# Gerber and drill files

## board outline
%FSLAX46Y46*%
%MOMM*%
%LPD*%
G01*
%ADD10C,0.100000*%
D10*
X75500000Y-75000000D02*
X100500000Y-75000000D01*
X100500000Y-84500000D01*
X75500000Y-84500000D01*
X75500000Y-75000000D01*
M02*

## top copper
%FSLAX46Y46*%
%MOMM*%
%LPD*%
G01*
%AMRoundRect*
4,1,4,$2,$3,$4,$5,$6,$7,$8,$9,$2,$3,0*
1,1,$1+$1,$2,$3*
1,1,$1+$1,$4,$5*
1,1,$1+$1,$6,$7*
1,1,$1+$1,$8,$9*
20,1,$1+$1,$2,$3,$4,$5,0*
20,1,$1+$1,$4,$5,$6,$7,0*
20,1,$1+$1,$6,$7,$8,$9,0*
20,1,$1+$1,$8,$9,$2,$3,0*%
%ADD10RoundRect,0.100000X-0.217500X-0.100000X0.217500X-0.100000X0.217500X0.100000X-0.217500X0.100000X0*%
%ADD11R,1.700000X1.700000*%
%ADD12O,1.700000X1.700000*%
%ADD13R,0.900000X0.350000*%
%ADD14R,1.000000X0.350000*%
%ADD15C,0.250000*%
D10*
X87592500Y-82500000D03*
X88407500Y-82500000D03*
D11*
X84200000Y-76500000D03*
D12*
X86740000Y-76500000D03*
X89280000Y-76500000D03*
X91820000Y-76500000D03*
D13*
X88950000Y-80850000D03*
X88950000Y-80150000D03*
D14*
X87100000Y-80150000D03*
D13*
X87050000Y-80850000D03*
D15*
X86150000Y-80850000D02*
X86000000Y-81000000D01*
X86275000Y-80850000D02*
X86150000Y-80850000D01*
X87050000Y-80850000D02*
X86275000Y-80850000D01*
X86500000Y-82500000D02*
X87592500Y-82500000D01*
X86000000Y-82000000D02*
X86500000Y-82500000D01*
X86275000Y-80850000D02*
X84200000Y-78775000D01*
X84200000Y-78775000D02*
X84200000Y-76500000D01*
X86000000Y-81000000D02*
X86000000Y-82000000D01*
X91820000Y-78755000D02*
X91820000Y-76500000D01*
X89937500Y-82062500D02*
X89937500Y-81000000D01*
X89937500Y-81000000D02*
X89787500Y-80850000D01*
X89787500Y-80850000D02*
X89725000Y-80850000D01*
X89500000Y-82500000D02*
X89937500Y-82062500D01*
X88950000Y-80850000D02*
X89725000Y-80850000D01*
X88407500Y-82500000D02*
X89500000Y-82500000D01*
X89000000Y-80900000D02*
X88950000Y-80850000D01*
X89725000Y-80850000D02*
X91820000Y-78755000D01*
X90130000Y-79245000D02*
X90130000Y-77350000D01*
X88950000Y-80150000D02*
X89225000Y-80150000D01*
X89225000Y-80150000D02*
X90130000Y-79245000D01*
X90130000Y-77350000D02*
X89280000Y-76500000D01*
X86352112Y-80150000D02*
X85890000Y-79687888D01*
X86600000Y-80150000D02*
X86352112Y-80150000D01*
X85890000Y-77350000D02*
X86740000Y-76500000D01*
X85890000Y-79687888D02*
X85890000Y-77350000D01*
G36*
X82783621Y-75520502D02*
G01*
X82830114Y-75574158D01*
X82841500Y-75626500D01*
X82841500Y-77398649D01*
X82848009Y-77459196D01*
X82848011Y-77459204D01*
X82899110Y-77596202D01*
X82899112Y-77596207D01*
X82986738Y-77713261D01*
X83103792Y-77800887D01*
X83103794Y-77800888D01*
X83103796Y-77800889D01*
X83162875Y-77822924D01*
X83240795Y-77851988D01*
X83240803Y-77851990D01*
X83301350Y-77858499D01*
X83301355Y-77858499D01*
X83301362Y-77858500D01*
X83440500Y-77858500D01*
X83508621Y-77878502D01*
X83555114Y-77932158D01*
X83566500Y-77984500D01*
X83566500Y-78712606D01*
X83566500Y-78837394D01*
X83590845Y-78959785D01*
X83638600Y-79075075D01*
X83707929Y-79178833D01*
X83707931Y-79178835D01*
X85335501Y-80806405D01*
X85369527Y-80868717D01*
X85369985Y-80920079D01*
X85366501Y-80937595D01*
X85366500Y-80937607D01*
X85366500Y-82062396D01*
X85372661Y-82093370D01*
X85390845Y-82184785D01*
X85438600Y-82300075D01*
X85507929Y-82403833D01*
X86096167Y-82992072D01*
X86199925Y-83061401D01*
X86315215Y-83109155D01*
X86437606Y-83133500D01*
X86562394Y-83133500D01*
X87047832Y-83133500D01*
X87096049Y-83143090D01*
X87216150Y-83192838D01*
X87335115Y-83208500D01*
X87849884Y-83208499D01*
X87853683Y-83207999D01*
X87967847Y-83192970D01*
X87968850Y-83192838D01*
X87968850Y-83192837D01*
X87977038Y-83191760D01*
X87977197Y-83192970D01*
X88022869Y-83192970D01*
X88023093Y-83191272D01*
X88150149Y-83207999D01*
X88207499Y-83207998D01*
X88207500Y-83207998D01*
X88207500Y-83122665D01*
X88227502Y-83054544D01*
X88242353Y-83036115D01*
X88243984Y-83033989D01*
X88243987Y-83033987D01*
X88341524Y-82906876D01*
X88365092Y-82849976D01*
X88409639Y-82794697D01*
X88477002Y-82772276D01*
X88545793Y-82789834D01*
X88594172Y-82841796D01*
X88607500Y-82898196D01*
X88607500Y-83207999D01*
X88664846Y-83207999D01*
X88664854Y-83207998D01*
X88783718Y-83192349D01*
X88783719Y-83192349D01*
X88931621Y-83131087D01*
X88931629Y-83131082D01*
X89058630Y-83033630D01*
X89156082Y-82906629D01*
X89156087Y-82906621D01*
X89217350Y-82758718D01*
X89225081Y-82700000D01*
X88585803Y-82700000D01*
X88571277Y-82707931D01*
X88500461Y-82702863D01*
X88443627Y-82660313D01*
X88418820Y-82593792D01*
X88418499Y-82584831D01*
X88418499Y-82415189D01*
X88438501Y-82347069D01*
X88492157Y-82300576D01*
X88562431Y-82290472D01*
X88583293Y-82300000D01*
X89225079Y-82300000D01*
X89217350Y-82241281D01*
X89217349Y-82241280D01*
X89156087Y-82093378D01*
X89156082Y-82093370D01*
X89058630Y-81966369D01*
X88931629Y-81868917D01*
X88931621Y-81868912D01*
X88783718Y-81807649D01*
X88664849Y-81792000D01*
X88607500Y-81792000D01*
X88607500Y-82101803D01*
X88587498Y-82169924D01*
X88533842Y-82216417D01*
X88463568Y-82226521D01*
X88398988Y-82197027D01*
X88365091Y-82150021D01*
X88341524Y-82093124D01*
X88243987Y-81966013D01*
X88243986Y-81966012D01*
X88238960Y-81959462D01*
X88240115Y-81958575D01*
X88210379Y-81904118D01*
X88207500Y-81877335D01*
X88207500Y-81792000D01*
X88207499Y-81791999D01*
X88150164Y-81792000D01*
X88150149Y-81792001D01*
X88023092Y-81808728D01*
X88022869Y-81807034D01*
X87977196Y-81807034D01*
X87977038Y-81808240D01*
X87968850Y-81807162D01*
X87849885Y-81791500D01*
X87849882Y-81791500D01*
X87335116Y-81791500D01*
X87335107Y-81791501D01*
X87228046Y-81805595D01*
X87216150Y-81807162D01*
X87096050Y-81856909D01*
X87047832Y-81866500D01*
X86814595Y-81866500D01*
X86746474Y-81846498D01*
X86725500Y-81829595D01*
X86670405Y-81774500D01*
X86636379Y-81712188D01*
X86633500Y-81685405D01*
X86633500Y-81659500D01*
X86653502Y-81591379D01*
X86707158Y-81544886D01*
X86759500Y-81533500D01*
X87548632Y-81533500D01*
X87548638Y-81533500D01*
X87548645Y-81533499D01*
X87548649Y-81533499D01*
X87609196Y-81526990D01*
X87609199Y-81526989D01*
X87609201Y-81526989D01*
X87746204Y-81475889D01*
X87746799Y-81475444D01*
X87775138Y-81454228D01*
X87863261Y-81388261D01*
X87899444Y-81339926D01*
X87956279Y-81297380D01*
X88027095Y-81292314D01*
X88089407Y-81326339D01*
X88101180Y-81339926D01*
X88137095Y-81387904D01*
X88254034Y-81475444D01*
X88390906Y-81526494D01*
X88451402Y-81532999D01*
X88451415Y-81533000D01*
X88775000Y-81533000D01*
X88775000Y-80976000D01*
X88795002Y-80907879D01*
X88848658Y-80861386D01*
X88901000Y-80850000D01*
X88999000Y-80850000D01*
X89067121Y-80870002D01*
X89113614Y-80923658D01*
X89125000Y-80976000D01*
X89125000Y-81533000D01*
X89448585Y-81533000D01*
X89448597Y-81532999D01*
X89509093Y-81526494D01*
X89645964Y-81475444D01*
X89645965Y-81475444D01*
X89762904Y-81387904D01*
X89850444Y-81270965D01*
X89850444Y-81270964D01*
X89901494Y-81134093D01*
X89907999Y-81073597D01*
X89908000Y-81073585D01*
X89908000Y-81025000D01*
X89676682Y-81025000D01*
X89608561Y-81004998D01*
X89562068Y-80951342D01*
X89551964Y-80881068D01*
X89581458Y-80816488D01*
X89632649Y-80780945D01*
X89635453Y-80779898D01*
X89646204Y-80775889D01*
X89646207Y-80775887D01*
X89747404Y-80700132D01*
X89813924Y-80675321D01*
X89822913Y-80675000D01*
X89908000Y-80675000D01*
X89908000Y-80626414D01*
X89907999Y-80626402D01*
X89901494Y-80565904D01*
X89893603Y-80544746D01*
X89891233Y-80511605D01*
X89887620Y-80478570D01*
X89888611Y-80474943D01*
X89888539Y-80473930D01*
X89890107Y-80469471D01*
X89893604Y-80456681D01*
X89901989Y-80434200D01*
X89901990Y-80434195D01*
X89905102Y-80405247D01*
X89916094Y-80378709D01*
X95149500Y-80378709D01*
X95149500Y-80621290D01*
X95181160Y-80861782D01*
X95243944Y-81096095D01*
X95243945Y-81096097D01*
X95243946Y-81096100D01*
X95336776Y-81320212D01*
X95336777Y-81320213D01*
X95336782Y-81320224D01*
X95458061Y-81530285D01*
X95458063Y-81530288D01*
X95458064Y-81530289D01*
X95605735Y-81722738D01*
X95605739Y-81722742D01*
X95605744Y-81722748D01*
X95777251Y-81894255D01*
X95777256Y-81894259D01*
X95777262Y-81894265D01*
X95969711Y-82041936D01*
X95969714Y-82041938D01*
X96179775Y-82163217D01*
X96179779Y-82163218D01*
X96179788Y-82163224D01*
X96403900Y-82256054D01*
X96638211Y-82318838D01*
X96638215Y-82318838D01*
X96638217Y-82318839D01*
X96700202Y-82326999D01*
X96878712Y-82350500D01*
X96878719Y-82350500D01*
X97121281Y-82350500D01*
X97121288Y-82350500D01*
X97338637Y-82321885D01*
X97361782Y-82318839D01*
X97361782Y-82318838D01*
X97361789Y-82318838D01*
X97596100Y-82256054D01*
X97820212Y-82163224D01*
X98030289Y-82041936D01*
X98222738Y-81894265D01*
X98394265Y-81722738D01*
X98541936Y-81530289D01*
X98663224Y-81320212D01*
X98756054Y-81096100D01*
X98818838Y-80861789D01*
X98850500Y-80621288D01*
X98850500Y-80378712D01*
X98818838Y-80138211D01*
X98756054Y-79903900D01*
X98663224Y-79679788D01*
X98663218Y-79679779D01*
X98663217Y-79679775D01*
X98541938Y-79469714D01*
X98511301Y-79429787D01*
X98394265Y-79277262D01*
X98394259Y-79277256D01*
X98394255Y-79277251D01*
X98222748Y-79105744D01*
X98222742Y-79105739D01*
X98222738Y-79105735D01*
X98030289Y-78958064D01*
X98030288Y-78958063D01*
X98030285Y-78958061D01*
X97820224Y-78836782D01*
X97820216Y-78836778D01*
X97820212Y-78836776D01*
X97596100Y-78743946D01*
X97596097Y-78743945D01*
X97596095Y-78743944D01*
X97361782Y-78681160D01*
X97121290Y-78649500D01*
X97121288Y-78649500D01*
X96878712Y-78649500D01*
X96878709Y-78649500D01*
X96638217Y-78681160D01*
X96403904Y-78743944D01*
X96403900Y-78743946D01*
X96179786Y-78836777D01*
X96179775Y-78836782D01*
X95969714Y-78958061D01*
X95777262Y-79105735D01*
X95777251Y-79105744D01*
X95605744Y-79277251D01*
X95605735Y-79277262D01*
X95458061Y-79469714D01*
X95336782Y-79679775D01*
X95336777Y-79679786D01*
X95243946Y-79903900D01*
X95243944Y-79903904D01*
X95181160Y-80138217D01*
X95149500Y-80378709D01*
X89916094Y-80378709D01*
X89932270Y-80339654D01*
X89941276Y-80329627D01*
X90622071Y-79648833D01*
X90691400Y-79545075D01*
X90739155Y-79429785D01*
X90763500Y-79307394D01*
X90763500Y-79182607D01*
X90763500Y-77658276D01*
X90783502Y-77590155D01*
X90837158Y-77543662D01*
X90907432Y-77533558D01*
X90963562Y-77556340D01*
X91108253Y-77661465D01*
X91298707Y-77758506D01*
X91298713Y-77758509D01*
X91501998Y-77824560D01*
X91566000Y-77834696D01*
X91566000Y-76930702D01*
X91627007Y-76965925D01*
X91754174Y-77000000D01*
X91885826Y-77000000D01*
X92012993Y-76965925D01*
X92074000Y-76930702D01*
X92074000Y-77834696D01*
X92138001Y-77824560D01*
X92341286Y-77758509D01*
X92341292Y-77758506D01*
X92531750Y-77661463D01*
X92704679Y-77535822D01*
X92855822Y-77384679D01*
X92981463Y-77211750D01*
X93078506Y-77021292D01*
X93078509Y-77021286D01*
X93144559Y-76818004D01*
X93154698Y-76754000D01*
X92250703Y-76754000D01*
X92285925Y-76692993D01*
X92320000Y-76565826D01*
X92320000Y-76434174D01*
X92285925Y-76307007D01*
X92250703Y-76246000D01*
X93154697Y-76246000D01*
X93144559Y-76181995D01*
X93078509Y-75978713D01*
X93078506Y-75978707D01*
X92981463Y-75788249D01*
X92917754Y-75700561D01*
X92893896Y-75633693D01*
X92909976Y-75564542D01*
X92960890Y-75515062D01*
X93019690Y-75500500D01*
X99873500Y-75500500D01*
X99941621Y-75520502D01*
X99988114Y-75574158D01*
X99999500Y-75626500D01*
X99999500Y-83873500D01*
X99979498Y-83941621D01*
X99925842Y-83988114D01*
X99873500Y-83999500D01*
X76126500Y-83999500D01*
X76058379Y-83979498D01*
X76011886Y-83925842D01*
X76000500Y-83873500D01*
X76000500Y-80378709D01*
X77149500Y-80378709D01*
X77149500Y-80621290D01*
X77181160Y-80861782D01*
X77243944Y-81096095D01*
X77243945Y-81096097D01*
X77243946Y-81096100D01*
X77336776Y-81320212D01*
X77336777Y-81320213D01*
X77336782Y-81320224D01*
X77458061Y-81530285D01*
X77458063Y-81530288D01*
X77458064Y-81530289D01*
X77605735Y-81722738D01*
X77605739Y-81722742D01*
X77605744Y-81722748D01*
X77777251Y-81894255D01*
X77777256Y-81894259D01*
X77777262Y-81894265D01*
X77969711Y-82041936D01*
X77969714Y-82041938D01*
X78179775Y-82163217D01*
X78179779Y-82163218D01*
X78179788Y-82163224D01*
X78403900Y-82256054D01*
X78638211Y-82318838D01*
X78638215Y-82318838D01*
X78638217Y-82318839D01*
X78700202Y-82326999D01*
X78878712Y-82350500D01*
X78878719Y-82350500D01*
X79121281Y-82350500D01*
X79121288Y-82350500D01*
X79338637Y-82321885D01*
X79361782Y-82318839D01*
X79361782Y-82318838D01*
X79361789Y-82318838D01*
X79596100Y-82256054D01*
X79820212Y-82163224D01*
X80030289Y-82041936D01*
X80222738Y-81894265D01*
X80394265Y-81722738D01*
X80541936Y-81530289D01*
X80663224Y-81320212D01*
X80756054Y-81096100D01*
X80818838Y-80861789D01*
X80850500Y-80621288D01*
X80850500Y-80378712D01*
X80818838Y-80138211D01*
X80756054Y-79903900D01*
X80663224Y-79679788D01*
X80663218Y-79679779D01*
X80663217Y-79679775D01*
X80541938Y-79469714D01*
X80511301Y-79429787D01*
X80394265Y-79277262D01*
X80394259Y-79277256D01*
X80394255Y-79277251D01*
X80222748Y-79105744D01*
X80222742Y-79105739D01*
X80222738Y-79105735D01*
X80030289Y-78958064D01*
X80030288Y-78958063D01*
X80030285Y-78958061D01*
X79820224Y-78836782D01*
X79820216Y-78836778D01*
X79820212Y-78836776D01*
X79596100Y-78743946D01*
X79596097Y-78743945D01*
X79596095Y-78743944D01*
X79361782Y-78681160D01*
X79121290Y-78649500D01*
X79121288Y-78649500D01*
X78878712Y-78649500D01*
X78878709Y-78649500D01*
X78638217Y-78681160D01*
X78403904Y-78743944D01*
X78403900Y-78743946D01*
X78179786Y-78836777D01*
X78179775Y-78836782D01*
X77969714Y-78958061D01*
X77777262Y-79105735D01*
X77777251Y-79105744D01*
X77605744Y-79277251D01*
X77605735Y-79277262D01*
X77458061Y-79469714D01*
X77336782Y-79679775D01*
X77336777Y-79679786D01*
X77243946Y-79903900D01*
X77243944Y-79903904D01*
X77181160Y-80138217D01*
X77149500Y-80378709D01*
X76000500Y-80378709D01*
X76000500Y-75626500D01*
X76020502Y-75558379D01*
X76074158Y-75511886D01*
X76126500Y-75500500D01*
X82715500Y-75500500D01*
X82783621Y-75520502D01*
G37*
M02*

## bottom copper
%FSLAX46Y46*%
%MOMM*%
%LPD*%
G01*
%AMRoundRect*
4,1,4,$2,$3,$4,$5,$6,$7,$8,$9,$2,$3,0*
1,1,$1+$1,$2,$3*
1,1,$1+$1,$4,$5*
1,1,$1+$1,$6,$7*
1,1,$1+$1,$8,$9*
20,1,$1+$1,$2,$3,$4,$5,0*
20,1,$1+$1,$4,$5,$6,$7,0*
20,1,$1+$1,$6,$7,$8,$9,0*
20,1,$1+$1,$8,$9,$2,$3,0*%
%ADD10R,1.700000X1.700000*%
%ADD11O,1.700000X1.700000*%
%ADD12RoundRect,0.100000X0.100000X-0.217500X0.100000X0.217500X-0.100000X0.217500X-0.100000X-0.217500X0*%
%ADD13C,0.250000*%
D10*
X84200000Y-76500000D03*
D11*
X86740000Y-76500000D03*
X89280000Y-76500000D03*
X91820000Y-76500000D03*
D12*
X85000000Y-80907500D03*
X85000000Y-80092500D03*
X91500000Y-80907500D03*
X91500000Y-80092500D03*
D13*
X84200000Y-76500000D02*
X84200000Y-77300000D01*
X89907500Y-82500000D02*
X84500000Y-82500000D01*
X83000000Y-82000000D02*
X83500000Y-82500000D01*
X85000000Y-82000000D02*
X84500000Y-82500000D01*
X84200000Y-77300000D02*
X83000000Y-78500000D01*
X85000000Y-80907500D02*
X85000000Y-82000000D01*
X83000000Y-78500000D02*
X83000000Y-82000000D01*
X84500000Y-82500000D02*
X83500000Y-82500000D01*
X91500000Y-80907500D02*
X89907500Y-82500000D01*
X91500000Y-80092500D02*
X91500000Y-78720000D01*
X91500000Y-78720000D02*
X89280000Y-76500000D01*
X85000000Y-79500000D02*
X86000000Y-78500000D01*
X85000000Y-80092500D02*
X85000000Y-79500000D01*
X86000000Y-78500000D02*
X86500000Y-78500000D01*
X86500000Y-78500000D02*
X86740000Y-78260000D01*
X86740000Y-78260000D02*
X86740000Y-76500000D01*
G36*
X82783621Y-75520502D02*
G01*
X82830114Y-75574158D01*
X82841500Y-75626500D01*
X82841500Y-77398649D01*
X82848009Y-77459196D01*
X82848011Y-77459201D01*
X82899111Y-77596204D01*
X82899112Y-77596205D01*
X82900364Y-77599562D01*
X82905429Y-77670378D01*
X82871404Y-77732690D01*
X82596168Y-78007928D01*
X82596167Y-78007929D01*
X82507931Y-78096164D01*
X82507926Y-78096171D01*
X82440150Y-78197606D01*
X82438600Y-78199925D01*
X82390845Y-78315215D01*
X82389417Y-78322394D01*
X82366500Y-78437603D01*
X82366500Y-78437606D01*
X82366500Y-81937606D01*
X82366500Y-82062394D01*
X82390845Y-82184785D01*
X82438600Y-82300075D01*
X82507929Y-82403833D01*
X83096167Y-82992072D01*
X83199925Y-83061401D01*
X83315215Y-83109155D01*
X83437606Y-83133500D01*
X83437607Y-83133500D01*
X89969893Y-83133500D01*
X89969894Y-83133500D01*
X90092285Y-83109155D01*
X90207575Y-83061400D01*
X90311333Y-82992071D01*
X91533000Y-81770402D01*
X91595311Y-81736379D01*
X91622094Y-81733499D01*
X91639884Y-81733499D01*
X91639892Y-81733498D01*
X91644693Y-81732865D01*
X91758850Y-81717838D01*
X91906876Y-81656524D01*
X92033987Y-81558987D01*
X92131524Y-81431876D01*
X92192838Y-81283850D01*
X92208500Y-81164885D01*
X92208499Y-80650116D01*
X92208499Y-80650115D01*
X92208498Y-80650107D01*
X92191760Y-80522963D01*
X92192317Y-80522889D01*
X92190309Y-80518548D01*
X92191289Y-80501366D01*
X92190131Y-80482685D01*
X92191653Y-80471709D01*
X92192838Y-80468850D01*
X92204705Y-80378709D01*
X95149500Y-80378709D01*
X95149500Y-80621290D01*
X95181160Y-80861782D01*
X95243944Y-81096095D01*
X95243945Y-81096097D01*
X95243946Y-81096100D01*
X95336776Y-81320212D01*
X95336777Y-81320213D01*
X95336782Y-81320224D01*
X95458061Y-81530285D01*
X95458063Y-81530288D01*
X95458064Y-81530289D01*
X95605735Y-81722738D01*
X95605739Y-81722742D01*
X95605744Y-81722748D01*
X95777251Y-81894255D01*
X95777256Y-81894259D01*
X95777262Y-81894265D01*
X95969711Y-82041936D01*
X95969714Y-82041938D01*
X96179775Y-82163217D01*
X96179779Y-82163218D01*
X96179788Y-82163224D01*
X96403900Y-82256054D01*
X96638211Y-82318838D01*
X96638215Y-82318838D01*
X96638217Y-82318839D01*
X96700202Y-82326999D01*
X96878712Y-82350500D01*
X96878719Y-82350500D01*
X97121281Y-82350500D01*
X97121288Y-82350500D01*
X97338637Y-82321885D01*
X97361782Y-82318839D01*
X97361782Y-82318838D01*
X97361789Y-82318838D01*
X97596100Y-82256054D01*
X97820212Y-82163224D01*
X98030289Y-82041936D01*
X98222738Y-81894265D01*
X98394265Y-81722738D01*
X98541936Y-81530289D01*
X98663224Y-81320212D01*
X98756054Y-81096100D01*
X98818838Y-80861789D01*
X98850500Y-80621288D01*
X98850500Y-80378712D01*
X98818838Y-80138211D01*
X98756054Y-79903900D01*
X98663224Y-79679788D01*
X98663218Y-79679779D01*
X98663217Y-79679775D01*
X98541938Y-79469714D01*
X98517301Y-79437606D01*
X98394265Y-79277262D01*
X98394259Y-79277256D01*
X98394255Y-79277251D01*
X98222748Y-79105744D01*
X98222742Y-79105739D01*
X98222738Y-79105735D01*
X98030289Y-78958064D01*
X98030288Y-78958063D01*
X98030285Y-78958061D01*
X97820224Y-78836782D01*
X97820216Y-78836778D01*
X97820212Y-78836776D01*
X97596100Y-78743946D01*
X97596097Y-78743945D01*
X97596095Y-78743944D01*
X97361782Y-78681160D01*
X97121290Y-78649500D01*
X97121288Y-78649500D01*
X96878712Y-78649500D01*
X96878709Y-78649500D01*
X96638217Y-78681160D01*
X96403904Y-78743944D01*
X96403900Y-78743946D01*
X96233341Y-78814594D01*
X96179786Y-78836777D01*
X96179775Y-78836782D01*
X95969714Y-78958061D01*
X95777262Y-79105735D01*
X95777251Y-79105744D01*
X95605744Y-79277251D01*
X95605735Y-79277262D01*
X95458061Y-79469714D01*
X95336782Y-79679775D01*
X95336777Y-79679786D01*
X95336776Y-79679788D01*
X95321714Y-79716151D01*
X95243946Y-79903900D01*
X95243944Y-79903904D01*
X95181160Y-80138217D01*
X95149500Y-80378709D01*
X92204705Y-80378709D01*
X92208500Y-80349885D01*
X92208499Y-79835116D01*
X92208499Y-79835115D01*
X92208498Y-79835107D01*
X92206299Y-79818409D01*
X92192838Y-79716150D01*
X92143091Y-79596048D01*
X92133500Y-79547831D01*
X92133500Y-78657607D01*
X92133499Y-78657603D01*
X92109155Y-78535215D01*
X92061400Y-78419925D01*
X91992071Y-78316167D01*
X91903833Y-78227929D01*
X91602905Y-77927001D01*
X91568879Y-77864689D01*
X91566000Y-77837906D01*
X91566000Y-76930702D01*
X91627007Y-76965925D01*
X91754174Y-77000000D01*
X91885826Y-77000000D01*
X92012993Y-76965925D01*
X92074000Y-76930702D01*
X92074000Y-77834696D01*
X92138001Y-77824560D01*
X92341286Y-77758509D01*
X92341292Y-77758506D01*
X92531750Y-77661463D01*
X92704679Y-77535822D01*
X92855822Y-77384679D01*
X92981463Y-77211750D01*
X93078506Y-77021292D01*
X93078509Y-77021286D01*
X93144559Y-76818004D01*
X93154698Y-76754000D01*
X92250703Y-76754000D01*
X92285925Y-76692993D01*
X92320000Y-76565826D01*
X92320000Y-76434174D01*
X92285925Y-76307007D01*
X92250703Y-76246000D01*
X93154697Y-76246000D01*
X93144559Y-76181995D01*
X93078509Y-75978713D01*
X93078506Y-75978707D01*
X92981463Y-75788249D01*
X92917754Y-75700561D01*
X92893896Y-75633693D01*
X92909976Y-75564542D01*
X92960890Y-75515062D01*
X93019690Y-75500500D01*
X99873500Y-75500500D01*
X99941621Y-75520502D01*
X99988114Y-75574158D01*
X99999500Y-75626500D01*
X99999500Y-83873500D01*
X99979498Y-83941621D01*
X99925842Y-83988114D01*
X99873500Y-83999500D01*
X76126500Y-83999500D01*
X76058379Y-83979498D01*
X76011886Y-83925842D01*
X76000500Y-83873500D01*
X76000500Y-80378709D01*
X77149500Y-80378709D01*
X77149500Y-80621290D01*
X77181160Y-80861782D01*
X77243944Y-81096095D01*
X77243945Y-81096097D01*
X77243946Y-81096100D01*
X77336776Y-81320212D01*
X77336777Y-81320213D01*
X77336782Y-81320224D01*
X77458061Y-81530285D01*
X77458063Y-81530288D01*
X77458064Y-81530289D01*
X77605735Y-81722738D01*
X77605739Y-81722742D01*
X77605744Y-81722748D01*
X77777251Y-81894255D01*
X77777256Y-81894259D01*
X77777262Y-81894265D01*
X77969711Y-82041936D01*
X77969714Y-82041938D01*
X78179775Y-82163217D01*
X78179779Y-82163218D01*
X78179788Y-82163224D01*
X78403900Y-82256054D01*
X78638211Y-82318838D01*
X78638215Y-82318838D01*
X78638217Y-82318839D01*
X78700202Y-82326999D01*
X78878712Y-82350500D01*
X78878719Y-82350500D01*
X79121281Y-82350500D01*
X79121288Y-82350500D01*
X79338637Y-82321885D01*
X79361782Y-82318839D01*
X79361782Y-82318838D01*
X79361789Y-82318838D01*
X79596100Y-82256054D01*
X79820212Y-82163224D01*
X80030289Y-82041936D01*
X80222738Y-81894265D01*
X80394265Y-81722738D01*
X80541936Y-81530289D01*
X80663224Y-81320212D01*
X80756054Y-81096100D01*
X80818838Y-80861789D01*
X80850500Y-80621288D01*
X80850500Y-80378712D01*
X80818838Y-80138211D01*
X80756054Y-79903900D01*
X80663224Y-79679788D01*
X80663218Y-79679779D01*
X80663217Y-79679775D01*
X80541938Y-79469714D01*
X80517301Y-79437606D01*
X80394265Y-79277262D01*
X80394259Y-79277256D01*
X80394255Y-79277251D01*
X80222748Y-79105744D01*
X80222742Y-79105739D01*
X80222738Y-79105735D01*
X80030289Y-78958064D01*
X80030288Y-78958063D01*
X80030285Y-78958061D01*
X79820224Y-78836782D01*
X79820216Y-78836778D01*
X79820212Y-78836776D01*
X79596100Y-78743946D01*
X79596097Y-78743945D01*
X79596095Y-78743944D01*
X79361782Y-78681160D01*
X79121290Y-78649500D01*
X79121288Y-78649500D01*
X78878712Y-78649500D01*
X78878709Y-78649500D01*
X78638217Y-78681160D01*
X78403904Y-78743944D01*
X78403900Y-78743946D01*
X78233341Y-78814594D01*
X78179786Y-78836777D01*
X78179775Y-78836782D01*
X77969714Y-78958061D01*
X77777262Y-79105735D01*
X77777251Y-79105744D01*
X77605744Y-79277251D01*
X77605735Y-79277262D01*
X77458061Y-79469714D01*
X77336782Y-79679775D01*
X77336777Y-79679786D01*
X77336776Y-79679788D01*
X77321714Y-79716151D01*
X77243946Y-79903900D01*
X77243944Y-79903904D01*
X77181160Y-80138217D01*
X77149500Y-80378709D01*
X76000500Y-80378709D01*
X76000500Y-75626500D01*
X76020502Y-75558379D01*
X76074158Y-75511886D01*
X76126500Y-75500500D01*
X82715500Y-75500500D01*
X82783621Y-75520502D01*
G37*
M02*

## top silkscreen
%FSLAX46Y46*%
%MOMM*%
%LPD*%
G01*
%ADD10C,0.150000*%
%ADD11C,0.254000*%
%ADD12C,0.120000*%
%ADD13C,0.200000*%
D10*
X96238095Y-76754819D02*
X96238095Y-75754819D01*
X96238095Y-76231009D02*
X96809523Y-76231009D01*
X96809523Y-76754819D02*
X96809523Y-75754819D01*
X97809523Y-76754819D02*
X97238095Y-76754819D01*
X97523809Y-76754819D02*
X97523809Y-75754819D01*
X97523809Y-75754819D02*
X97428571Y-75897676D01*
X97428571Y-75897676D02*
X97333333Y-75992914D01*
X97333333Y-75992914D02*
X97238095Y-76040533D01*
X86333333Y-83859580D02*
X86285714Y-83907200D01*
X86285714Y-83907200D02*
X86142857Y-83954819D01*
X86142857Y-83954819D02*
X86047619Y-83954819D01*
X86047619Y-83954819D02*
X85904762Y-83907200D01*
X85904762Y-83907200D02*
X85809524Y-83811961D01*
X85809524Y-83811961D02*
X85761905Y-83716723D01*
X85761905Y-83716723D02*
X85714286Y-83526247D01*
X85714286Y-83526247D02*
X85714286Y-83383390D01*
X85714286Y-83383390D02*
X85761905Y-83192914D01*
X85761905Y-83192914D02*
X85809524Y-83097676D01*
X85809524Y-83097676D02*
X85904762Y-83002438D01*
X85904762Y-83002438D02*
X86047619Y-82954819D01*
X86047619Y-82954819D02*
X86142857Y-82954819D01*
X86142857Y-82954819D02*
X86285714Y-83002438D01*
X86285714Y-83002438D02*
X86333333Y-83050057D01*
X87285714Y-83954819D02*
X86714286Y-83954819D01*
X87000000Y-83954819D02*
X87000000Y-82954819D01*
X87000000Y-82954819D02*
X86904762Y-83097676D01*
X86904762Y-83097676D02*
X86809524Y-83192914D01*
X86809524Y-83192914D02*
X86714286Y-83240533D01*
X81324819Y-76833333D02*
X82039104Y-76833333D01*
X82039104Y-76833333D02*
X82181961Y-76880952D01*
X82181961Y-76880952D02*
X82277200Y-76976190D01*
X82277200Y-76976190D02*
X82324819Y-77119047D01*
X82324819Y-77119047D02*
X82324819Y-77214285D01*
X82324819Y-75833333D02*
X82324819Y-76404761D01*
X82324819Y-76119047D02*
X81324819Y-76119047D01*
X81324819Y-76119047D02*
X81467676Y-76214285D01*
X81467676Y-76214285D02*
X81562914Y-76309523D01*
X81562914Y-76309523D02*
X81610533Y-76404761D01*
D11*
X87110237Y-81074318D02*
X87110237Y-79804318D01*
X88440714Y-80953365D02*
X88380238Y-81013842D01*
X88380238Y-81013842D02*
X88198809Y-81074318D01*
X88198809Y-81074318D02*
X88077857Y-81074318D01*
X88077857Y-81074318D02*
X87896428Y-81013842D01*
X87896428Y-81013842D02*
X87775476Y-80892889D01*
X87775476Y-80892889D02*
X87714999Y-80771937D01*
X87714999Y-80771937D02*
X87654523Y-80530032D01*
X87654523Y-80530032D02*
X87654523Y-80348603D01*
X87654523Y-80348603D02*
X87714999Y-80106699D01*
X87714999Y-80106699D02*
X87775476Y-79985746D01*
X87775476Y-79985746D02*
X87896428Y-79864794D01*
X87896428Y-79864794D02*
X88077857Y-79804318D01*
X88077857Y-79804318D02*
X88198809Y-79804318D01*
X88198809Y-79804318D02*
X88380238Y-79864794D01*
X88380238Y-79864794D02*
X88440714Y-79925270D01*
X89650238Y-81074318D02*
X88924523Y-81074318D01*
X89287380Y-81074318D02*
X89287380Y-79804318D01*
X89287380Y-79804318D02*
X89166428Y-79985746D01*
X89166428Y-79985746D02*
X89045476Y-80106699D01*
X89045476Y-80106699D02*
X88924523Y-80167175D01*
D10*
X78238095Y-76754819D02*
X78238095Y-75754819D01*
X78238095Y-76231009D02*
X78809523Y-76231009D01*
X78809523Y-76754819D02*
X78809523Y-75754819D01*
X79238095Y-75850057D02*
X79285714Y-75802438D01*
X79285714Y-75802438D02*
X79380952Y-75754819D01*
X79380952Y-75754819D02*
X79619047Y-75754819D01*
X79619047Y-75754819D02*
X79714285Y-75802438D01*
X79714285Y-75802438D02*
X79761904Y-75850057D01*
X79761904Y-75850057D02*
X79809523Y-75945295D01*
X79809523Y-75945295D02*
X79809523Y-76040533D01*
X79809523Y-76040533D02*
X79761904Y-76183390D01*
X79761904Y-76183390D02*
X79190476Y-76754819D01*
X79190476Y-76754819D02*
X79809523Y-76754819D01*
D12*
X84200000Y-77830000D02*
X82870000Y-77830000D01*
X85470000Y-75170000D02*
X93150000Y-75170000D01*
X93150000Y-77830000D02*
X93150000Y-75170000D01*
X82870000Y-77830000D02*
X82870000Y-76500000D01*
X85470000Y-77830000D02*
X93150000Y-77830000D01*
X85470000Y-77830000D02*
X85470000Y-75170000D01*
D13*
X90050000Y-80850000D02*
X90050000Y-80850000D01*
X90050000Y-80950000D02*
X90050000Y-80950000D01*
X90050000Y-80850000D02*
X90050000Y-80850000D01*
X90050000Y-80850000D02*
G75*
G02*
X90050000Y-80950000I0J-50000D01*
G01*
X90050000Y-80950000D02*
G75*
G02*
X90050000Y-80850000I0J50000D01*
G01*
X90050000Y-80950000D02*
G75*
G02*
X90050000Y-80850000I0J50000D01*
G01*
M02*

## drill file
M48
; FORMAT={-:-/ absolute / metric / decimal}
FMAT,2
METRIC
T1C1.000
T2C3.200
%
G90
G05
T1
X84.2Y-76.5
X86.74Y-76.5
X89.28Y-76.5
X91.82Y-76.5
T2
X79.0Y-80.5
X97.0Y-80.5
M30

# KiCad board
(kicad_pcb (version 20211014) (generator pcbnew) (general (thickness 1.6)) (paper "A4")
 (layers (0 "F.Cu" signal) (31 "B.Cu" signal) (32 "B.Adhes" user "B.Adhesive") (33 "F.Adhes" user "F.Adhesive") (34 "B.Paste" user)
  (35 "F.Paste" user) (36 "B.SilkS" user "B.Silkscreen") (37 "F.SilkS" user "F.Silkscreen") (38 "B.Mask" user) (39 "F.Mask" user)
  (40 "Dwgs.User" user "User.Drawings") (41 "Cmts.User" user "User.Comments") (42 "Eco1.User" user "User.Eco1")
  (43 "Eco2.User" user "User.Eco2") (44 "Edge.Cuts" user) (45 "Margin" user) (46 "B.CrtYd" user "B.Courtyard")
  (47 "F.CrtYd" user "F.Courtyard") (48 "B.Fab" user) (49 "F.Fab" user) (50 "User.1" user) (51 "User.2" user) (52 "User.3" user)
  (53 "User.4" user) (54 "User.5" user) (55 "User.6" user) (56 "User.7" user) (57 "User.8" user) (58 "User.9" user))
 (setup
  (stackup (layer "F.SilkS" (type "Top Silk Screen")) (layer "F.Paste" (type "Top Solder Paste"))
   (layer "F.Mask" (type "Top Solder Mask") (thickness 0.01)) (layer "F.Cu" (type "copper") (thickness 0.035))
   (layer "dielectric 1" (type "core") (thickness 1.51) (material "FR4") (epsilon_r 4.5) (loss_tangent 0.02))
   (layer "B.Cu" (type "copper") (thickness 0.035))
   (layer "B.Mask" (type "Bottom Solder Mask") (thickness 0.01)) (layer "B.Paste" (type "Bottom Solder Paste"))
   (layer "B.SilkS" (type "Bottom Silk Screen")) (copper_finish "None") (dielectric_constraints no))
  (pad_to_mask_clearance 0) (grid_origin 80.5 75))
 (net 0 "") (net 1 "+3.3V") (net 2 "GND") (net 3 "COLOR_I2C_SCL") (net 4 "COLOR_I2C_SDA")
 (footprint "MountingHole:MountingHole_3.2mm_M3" (layer "F.Cu") (at 97 80.5)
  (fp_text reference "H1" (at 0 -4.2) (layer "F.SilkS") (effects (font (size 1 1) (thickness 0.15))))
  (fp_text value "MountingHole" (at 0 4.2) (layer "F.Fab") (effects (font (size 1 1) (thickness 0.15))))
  (pad "" np_thru_hole circle (at 0 0) (size 3.2 3.2) (drill 3.2) (layers *.Cu *.Mask)))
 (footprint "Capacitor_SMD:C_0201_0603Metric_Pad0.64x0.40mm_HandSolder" (layer "F.Cu") (at 88 82.5)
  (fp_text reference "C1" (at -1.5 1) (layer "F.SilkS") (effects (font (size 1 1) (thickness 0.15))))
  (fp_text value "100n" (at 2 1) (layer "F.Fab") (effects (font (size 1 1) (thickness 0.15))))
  (pad "" smd roundrect (at 0.4325 0) (size 0.458 0.36) (layers "F.Paste") (roundrect_rratio 0.25))
  (pad "" smd roundrect (at -0.4325 0) (size 0.458 0.36) (layers "F.Paste") (roundrect_rratio 0.25))
  (pad "1" smd roundrect (at -0.4075 0) (size 0.635 0.4) (layers "F.Cu" "F.Mask") (roundrect_rratio 0.25) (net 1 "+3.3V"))
  (pad "2" smd roundrect (at 0.4075 0) (size 0.635 0.4) (layers "F.Cu" "F.Mask") (roundrect_rratio 0.25) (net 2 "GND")))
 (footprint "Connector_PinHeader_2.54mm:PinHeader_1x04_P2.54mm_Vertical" (layer "F.Cu") (at 84.2 76.5 90)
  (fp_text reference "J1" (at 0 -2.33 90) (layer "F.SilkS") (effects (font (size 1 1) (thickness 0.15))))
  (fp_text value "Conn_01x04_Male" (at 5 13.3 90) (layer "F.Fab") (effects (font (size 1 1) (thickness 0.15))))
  (fp_line (start -1.33 0) (end -1.33 -1.33) (layer "F.SilkS") (width 0.12))
  (fp_line (start 1.33 1.27) (end 1.33 8.95) (layer "F.SilkS") (width 0.12))
  (fp_line (start -1.33 8.95) (end 1.33 8.95) (layer "F.SilkS") (width 0.12))
  (fp_line (start -1.33 -1.33) (end 0 -1.33) (layer "F.SilkS") (width 0.12))
  (fp_line (start -1.33 1.27) (end -1.33 8.95) (layer "F.SilkS") (width 0.12))
  (fp_line (start -1.33 1.27) (end 1.33 1.27) (layer "F.SilkS") (width 0.12))
  (pad "1" thru_hole rect (at 0 0 90) (size 1.7 1.7) (drill 1) (layers *.Cu *.Mask) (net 1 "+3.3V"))
  (pad "2" thru_hole oval (at 0 2.54 90) (size 1.7 1.7) (drill 1) (layers *.Cu *.Mask) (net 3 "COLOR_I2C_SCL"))
  (pad "3" thru_hole oval (at 0 5.08 90) (size 1.7 1.7) (drill 1) (layers *.Cu *.Mask) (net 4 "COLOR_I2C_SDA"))
  (pad "4" thru_hole oval (at 0 7.62 90) (size 1.7 1.7) (drill 1) (layers *.Cu *.Mask) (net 2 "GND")))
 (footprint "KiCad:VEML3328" (layer "F.Cu") (at 88 80.5 180)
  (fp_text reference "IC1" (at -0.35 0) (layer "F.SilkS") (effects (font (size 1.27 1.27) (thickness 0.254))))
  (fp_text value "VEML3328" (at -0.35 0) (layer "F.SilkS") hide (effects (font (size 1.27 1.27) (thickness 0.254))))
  (fp_line (start -2.05 -0.35) (end -2.05 -0.35) (layer "F.SilkS") (width 0.2))
  (fp_line (start -2.05 -0.45) (end -2.05 -0.45) (layer "F.SilkS") (width 0.2))
  (fp_line (start -2.05 -0.35) (end -2.05 -0.35) (layer "F.SilkS") (width 0.2))
  (fp_arc (start -2.05 -0.35) (mid -2.1 -0.4) (end -2.05 -0.45) (layer "F.SilkS") (width 0.2))
  (fp_arc (start -2.05 -0.45) (mid -2 -0.4) (end -2.05 -0.35) (layer "F.SilkS") (width 0.2))
  (fp_arc (start -2.05 -0.45) (mid -2 -0.4) (end -2.05 -0.35) (layer "F.SilkS") (width 0.2))
  (pad "1" smd rect locked (at -0.95 -0.35 270) (size 0.35 0.9) (layers "F.Cu" "F.Paste" "F.Mask") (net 2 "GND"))
  (pad "2" smd rect locked (at -0.95 0.35 270) (size 0.35 0.9) (layers "F.Cu" "F.Paste" "F.Mask") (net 4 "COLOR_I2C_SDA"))
  (pad "3" smd rect locked (at 0.9 0.35 270) (size 0.35 1) (layers "F.Cu" "F.Paste" "F.Mask") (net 3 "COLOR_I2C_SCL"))
  (pad "4" smd rect locked (at 0.95 -0.35 270) (size 0.35 0.9) (layers "F.Cu" "F.Paste" "F.Mask") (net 1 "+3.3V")))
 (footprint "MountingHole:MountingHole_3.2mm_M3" (layer "F.Cu") (at 79 80.5)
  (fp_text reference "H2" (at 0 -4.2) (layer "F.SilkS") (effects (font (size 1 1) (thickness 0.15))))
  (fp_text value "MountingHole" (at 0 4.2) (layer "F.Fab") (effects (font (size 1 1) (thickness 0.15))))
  (pad "" np_thru_hole circle (at 0 0) (size 3.2 3.2) (drill 3.2) (layers *.Cu *.Mask)))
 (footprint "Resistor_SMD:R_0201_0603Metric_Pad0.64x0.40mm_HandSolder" (layer "B.Cu") (at 85 80.5 90)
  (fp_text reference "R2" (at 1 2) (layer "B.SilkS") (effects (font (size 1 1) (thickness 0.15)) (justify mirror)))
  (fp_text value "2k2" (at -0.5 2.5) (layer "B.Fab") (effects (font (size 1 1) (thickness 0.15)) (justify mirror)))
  (pad "" smd roundrect (at -0.4325 0 90) (size 0.458 0.36) (layers "B.Paste") (roundrect_rratio 0.25))
  (pad "" smd roundrect (at 0.4325 0 90) (size 0.458 0.36) (layers "B.Paste") (roundrect_rratio 0.25))
  (pad "1" smd roundrect (at -0.4075 0 90) (size 0.635 0.4) (layers "B.Cu" "B.Mask") (roundrect_rratio 0.25) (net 1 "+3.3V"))
  (pad "2" smd roundrect (at 0.4075 0 90) (size 0.635 0.4) (layers "B.Cu" "B.Mask") (roundrect_rratio 0.25) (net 3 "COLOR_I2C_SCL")))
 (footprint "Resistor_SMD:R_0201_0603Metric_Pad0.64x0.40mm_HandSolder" (layer "B.Cu") (at 91.5 80.5 90)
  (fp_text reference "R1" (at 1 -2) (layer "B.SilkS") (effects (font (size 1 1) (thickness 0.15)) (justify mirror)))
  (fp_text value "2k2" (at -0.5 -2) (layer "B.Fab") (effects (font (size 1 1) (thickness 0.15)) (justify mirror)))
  (pad "" smd roundrect (at -0.4325 0 90) (size 0.458 0.36) (layers "B.Paste") (roundrect_rratio 0.25))
  (pad "" smd roundrect (at 0.4325 0 90) (size 0.458 0.36) (layers "B.Paste") (roundrect_rratio 0.25))
  (pad "1" smd roundrect (at -0.4075 0 90) (size 0.635 0.4) (layers "B.Cu" "B.Mask") (roundrect_rratio 0.25) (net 1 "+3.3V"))
  (pad "2" smd roundrect (at 0.4075 0 90) (size 0.635 0.4) (layers "B.Cu" "B.Mask") (roundrect_rratio 0.25) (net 4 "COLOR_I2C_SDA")))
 (gr_rect (start 75.5 75) (end 100.5 84.5) (layer "Edge.Cuts") (width 0.1) (fill none))
 (segment (start 86.15 80.85) (end 86 81) (width 0.25) (layer "F.Cu") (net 1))
 (segment (start 86.275 80.85) (end 86.15 80.85) (width 0.25) (layer "F.Cu") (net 1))
 (segment (start 87.05 80.85) (end 86.275 80.85) (width 0.25) (layer "F.Cu") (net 1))
 (segment (start 86.5 82.5) (end 87.5925 82.5) (width 0.25) (layer "F.Cu") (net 1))
 (segment (start 86 82) (end 86.5 82.5) (width 0.25) (layer "F.Cu") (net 1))
 (segment (start 86.275 80.85) (end 84.2 78.775) (width 0.25) (layer "F.Cu") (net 1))
 (segment (start 84.2 78.775) (end 84.2 76.5) (width 0.25) (layer "F.Cu") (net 1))
 (segment (start 86 81) (end 86 82) (width 0.25) (layer "F.Cu") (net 1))
 (segment (start 84.2 76.5) (end 84.2 77.3) (width 0.25) (layer "B.Cu") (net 1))
 (segment (start 89.9075 82.5) (end 84.5 82.5) (width 0.25) (layer "B.Cu") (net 1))
 (segment (start 83 82) (end 83.5 82.5) (width 0.25) (layer "B.Cu") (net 1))
 (segment (start 85 82) (end 84.5 82.5) (width 0.25) (layer "B.Cu") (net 1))
 (segment (start 84.2 77.3) (end 83 78.5) (width 0.25) (layer "B.Cu") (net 1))
 (segment (start 85 80.9075) (end 85 82) (width 0.25) (layer "B.Cu") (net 1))
 (segment (start 83 78.5) (end 83 82) (width 0.25) (layer "B.Cu") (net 1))
 (segment (start 84.5 82.5) (end 83.5 82.5) (width 0.25) (layer "B.Cu") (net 1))
 (segment (start 91.5 80.9075) (end 89.9075 82.5) (width 0.25) (layer "B.Cu") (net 1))
 (segment (start 91.82 78.755) (end 91.82 76.5) (width 0.25) (layer "F.Cu") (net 2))
 (segment (start 89.9375 82.0625) (end 89.9375 81) (width 0.25) (layer "F.Cu") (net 2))
 (segment (start 89.9375 81) (end 89.7875 80.85) (width 0.25) (layer "F.Cu") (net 2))
 (segment (start 89.7875 80.85) (end 89.725 80.85) (width 0.25) (layer "F.Cu") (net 2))
 (segment (start 89.5 82.5) (end 89.9375 82.0625) (width 0.25) (layer "F.Cu") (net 2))
 (segment (start 88.95 80.85) (end 89.725 80.85) (width 0.25) (layer "F.Cu") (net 2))
 (segment (start 88.4075 82.5) (end 89.5 82.5) (width 0.25) (layer "F.Cu") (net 2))
 (segment (start 89 80.9) (end 88.95 80.85) (width 0.25) (layer "F.Cu") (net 2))
 (segment (start 89.725 80.85) (end 91.82 78.755) (width 0.25) (layer "F.Cu") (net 2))
 (segment (start 90.13 79.245) (end 90.13 77.35) (width 0.25) (layer "F.Cu") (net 4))
 (segment (start 88.95 80.15) (end 89.225 80.15) (width 0.25) (layer "F.Cu") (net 4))
 (segment (start 89.225 80.15) (end 90.13 79.245) (width 0.25) (layer "F.Cu") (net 4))
 (segment (start 90.13 77.35) (end 89.28 76.5) (width 0.25) (layer "F.Cu") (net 4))
 (segment (start 91.5 80.0925) (end 91.5 78.72) (width 0.25) (layer "B.Cu") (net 4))
 (segment (start 91.5 78.72) (end 89.28 76.5) (width 0.25) (layer "B.Cu") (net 4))
 (segment (start 86.352112 80.15) (end 85.89 79.687888) (width 0.25) (layer "F.Cu") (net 3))
 (segment (start 86.6 80.15) (end 86.352112 80.15) (width 0.25) (layer "F.Cu") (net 3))
 (segment (start 85.89 77.35) (end 86.74 76.5) (width 0.25) (layer "F.Cu") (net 3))
 (segment (start 85.89 79.687888) (end 85.89 77.35) (width 0.25) (layer "F.Cu") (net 3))
 (segment (start 85 79.5) (end 86 78.5) (width 0.25) (layer "B.Cu") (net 3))
 (segment (start 85 80.0925) (end 85 79.5) (width 0.25) (layer "B.Cu") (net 3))
 (segment (start 86 78.5) (end 86.5 78.5) (width 0.25) (layer "B.Cu") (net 3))
 (segment (start 86.5 78.5) (end 86.74 78.26) (width 0.25) (layer "B.Cu") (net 3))
 (segment (start 86.74 78.26) (end 86.74 76.5) (width 0.25) (layer "B.Cu") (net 3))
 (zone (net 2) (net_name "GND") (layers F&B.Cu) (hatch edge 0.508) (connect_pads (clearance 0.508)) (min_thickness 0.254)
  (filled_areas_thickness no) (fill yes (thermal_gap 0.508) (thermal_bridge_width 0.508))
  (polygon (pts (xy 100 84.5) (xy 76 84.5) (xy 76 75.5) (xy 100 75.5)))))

